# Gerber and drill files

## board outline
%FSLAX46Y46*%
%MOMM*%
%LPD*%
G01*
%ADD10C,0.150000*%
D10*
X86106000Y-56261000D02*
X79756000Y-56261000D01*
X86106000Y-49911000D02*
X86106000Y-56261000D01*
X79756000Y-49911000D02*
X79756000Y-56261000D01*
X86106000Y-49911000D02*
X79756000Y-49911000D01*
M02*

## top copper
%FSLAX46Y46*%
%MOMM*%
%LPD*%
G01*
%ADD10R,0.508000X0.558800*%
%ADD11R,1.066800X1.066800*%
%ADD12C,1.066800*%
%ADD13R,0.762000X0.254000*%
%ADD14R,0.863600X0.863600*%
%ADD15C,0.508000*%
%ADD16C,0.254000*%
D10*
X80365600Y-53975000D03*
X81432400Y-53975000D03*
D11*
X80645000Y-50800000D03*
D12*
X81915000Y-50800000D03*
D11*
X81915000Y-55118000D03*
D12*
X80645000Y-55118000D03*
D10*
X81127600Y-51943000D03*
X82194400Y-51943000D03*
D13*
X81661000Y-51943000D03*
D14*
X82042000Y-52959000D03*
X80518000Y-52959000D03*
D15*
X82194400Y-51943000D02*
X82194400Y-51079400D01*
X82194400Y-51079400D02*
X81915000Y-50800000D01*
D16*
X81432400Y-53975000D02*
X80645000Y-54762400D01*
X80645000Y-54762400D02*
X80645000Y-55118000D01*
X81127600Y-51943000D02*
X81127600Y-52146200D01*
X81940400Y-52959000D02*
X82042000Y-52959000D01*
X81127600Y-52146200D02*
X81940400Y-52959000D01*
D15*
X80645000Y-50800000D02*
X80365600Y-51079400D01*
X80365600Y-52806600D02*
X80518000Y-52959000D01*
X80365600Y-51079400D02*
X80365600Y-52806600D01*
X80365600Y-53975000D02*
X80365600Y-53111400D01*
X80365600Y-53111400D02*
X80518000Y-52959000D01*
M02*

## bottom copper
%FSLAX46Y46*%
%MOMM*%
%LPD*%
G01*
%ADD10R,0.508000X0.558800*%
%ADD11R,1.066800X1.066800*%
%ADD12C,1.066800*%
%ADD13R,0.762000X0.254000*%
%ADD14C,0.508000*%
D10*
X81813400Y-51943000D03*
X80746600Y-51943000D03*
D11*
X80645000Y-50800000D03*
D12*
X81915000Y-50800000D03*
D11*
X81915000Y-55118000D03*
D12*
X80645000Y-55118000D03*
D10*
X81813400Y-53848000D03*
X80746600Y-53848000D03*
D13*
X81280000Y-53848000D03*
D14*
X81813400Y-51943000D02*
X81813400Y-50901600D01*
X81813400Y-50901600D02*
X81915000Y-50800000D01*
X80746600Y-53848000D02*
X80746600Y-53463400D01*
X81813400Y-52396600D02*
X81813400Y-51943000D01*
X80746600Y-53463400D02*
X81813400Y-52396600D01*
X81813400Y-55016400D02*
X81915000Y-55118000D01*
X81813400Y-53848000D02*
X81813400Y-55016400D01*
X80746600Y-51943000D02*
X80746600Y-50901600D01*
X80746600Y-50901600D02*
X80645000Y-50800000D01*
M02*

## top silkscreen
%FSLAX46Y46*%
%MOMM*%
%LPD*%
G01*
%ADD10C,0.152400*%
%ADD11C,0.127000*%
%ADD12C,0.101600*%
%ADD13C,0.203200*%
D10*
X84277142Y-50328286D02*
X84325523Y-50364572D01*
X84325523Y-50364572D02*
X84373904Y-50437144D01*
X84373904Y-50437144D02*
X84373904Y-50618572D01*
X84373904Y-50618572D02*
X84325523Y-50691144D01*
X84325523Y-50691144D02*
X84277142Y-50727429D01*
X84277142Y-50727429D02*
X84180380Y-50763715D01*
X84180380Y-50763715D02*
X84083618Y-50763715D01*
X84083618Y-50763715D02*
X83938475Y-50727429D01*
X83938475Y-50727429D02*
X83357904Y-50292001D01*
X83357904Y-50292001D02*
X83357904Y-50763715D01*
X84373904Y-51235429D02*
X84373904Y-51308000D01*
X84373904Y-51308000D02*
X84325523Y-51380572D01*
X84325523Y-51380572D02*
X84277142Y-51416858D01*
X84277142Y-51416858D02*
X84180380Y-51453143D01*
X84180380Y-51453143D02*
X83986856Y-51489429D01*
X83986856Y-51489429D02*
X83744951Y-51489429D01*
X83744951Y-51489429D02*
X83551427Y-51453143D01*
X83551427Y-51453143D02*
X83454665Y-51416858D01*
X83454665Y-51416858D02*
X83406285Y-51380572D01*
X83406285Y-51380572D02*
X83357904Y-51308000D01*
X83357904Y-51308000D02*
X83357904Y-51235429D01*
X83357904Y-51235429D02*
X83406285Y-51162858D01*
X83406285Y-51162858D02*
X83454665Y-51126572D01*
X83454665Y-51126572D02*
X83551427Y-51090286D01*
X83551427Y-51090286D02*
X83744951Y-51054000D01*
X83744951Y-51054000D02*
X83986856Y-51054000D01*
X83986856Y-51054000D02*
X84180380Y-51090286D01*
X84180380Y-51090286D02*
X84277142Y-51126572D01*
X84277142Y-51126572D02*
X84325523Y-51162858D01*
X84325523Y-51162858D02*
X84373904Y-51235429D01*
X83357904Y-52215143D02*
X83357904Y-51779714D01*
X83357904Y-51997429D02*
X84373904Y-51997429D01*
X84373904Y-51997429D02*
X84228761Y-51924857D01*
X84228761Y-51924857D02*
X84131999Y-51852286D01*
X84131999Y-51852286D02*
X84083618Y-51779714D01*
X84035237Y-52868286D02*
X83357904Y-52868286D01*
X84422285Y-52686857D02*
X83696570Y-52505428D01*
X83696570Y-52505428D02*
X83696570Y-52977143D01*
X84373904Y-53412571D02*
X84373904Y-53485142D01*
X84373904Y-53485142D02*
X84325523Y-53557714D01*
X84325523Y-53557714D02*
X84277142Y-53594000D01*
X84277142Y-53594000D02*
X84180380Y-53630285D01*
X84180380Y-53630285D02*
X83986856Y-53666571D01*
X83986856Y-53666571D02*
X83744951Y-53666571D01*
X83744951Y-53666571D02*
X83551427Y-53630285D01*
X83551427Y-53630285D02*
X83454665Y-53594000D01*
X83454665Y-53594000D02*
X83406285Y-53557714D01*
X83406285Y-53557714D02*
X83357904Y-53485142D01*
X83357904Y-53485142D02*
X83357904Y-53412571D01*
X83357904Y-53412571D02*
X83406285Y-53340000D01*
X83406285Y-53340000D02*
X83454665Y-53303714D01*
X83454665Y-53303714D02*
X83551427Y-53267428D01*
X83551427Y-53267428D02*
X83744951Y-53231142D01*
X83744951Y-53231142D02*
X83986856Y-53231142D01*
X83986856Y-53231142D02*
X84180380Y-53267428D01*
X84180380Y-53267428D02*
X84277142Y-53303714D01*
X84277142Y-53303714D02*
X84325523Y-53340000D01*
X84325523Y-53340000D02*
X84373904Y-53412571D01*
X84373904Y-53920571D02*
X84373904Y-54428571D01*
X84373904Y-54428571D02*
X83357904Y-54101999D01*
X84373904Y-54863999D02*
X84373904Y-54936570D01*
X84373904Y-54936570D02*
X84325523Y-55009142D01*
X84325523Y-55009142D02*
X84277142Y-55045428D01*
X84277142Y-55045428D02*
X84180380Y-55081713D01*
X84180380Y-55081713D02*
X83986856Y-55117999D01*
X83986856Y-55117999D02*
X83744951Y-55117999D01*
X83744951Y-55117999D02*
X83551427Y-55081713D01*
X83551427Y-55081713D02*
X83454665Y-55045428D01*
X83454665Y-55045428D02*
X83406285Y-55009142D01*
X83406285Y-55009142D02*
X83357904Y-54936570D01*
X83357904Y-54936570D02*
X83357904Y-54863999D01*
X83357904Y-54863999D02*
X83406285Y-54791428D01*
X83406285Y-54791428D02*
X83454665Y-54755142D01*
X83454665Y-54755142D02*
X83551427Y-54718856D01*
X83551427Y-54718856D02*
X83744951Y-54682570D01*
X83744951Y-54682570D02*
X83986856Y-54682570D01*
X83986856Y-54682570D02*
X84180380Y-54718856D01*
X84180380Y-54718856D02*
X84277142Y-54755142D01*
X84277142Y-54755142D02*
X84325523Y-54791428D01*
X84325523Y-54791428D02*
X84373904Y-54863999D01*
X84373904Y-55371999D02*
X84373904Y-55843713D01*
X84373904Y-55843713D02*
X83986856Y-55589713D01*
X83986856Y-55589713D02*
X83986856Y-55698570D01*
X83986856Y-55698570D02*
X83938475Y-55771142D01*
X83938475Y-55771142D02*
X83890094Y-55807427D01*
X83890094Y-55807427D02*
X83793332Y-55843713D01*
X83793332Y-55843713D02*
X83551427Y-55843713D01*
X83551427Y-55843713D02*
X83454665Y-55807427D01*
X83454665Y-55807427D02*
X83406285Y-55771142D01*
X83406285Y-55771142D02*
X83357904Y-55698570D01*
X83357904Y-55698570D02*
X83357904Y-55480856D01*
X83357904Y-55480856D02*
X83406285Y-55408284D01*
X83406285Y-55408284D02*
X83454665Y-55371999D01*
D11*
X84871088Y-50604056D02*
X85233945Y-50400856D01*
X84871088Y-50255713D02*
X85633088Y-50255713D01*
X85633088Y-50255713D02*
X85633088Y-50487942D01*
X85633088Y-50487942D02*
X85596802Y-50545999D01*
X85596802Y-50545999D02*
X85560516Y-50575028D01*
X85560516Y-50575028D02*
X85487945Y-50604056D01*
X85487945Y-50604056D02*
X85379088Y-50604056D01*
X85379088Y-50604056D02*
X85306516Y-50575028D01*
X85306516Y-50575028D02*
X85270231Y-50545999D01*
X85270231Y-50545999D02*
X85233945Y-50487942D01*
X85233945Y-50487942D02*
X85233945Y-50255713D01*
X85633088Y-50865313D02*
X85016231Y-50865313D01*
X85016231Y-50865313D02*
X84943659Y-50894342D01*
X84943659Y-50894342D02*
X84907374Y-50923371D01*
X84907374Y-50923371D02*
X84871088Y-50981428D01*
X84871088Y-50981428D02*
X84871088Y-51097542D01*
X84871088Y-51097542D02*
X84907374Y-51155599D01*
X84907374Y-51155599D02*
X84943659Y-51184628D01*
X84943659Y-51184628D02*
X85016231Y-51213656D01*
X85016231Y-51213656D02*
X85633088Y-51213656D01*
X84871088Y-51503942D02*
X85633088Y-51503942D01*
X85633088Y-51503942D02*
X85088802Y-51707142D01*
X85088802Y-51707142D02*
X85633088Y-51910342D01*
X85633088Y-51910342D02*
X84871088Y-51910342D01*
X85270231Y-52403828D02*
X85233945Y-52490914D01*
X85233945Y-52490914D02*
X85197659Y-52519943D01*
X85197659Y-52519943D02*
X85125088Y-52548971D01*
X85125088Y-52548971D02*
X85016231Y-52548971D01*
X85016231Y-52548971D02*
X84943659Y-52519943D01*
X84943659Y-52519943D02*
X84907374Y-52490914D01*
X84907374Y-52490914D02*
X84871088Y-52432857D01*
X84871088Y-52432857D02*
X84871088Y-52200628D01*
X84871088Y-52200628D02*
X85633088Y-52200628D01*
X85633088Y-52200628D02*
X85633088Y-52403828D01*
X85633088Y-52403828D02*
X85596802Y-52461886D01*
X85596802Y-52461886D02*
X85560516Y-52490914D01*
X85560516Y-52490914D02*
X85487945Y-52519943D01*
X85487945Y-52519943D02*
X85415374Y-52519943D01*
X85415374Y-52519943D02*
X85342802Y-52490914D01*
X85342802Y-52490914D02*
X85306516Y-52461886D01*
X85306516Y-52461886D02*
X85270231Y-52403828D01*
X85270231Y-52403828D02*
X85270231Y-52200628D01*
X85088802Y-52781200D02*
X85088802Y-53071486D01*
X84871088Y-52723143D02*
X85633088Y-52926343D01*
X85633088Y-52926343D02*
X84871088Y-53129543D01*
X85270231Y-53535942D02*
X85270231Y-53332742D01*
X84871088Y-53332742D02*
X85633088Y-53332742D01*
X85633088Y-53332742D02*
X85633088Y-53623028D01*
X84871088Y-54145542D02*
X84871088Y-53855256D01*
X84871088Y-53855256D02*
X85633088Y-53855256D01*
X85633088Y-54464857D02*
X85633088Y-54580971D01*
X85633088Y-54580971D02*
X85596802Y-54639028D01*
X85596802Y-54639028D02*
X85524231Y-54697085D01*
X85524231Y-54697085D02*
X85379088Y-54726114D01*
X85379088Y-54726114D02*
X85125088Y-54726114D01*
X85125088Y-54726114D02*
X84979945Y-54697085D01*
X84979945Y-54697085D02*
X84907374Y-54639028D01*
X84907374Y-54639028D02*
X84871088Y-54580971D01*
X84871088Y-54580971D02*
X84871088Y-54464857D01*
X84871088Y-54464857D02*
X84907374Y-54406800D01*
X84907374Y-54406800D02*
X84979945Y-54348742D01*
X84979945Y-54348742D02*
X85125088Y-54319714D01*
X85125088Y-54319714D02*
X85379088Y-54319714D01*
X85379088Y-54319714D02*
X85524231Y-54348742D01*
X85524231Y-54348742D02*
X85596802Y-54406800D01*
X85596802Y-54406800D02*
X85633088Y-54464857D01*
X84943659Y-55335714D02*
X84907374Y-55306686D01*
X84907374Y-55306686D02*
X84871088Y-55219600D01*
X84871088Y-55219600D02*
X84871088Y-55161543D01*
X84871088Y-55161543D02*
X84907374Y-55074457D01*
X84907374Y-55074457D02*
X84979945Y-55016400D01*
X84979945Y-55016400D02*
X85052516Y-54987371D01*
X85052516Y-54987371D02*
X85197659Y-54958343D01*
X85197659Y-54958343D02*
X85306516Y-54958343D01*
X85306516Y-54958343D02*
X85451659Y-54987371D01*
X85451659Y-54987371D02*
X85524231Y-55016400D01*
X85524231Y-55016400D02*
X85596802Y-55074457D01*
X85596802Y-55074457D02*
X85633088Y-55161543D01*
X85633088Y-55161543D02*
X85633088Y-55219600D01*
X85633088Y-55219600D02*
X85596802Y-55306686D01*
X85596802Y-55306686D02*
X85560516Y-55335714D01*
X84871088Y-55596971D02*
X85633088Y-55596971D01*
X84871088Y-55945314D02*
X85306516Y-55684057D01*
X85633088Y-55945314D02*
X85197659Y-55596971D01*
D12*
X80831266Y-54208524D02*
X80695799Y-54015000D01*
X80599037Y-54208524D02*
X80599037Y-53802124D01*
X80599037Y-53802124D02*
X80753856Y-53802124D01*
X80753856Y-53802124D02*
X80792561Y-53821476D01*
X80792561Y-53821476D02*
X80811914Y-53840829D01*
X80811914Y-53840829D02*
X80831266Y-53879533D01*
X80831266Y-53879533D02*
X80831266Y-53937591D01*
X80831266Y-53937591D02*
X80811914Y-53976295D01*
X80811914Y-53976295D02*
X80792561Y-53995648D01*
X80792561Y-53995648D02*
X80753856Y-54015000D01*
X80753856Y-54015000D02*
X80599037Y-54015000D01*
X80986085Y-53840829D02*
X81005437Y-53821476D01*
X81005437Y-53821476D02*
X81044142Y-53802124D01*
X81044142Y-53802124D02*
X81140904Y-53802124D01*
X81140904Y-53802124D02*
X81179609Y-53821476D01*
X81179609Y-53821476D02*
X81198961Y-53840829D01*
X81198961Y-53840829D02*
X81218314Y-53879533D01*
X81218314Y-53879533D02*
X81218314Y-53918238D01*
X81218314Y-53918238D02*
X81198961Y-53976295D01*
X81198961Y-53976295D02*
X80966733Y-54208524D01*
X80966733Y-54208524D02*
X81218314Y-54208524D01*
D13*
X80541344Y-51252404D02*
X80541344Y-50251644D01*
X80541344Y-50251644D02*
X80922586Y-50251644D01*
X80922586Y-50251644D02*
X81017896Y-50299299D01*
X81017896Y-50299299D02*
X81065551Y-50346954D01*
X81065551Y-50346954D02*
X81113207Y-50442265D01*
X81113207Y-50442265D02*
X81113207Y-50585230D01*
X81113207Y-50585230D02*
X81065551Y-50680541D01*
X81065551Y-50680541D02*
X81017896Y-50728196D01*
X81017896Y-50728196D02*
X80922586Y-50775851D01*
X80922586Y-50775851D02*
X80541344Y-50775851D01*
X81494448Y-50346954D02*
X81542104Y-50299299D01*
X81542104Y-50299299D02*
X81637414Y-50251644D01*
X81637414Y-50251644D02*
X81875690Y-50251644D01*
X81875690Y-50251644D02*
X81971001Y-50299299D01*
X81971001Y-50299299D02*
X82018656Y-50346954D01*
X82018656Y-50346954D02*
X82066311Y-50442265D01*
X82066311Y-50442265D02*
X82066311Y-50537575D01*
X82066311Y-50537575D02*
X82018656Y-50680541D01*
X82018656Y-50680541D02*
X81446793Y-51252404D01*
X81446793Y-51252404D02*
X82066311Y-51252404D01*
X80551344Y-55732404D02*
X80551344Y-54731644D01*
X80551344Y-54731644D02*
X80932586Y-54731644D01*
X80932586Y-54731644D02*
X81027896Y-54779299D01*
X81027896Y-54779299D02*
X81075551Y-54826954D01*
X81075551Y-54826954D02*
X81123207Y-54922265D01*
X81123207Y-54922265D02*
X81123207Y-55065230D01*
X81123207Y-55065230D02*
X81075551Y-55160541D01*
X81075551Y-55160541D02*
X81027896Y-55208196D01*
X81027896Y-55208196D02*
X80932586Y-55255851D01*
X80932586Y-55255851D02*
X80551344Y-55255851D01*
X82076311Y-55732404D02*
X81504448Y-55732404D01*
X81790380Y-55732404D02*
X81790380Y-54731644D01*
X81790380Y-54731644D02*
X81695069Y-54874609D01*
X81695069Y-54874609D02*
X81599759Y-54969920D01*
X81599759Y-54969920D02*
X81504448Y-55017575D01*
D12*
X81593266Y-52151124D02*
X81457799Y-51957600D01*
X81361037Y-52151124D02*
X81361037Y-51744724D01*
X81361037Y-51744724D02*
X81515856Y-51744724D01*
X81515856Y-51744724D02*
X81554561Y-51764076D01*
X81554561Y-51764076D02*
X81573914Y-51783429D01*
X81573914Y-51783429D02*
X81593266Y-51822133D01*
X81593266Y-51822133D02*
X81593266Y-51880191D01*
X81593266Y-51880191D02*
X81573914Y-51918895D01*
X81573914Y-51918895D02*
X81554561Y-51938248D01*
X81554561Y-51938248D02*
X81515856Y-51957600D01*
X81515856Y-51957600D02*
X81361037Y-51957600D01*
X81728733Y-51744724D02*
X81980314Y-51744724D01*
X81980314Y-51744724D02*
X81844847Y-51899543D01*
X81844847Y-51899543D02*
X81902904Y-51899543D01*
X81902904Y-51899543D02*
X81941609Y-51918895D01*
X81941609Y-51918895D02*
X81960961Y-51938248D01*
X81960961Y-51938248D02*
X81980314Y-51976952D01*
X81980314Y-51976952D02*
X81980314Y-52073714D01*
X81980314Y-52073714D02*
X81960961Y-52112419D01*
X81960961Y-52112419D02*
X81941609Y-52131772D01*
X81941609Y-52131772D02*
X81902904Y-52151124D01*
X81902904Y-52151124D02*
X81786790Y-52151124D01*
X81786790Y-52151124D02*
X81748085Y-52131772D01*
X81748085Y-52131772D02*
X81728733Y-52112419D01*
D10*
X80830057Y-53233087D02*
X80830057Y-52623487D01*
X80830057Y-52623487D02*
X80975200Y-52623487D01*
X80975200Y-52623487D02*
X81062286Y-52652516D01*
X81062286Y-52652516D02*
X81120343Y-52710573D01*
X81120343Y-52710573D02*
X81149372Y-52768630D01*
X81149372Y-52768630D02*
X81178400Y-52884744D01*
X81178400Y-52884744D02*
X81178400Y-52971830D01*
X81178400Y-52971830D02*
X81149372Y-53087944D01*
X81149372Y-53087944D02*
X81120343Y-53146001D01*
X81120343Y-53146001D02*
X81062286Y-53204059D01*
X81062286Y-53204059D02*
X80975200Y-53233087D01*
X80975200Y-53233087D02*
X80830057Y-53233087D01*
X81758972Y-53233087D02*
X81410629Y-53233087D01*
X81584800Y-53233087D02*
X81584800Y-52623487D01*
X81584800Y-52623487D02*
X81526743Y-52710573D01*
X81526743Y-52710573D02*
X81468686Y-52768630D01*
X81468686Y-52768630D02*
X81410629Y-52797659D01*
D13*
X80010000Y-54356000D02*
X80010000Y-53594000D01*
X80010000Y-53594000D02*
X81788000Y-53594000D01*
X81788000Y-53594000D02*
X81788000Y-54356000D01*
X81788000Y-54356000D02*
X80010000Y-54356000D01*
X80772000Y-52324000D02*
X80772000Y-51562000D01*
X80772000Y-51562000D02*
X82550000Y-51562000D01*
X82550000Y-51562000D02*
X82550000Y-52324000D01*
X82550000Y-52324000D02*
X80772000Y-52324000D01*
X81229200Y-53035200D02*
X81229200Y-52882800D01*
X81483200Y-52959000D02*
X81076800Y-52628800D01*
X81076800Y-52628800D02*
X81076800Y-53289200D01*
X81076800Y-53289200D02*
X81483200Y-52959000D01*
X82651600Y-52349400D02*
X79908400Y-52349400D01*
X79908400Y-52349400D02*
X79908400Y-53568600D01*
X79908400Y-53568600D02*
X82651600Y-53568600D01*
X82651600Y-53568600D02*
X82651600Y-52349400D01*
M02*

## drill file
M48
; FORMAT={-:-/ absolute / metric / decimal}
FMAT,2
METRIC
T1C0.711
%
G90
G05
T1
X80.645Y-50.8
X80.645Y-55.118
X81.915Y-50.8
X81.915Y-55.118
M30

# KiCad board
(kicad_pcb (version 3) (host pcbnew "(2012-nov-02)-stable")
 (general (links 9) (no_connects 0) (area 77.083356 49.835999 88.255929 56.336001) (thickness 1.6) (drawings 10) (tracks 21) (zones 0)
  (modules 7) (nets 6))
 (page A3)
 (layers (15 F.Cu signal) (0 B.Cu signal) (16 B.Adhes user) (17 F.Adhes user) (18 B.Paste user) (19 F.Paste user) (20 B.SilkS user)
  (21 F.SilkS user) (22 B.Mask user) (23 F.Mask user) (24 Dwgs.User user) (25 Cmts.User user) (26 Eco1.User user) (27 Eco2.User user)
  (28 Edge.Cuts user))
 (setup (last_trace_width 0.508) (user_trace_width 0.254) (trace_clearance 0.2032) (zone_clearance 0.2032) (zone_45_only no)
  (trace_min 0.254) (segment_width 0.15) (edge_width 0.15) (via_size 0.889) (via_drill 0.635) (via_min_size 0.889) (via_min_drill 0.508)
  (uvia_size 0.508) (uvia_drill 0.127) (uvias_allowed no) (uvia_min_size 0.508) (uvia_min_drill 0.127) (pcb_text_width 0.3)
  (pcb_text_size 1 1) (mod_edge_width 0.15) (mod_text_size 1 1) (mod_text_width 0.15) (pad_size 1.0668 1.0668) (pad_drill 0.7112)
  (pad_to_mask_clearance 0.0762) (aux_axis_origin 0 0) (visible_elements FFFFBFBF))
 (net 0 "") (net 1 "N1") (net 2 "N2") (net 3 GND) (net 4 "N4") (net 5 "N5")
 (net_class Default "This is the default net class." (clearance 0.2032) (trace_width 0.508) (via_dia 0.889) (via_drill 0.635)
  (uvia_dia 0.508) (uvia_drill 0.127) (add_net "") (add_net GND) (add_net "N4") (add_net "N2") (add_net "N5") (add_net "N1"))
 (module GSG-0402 (layer F.Cu) (at 80.899 53.975 180) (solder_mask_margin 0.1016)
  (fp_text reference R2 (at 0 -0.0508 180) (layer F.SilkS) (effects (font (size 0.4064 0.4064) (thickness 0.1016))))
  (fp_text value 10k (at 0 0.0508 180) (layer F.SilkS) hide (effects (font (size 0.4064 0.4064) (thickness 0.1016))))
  (fp_line (start 0.889 -0.381) (end 0.889 0.381) (layer F.SilkS) (width 0.2032))
  (fp_line (start 0.889 0.381) (end -0.889 0.381) (layer F.SilkS) (width 0.2032))
  (fp_line (start -0.889 0.381) (end -0.889 -0.381) (layer F.SilkS) (width 0.2032))
  (fp_line (start -0.889 -0.381) (end 0.889 -0.381) (layer F.SilkS) (width 0.2032))
  (pad 2 smd rect (at 0.5334 0 180) (size 0.508 0.5588) (layers F.Cu F.Paste F.Mask) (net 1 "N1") (solder_mask_margin 0.1016))
  (pad 1 smd rect (at -0.5334 0 180) (size 0.508 0.5588) (layers F.Cu F.Paste F.Mask) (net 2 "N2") (die_length -2147.483648)
   (solder_mask_margin 0.1016)))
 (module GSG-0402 (layer B.Cu) (at 81.28 51.943) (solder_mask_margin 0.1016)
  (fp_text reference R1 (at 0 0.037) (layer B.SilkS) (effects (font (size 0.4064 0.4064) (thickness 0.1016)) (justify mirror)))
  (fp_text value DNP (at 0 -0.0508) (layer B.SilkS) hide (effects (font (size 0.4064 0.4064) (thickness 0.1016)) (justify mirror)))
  (pad 2 smd rect (at 0.5334 0) (size 0.508 0.5588) (layers B.Cu B.Paste B.Mask) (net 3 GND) (solder_mask_margin 0.1016))
  (pad 1 smd rect (at -0.5334 0) (size 0.508 0.5588) (layers B.Cu B.Paste B.Mask) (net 1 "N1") (die_length -2147.483648)
   (solder_mask_margin 0.1016)))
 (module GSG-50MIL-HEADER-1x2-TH (layer F.Cu) (at 81.28 50.8)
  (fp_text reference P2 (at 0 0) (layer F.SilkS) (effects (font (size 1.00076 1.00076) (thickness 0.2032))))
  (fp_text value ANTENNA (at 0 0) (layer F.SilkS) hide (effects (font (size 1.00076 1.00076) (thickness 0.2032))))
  (pad 1 thru_hole rect (at -0.635 0) (size 1.0668 1.0668) (drill 0.7112) (layers *.Cu *.Mask) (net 1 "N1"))
  (pad 2 thru_hole circle (at 0.635 0) (size 1.0668 1.0668) (drill 0.7112) (layers *.Cu *.Mask) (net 3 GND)))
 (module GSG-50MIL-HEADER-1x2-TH (layer F.Cu) (at 81.28 55.118 180)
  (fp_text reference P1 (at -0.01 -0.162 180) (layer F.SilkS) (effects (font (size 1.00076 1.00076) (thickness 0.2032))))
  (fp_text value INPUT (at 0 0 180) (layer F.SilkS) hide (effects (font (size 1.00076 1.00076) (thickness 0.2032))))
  (pad 1 thru_hole rect (at -0.635 0 180) (size 1.0668 1.0668) (drill 0.7112) (layers *.Cu *.Mask) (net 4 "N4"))
  (pad 2 thru_hole circle (at 0.635 0 180) (size 1.0668 1.0668) (drill 0.7112) (layers *.Cu *.Mask) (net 2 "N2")))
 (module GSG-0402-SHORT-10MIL (layer B.Cu) (at 81.28 53.848) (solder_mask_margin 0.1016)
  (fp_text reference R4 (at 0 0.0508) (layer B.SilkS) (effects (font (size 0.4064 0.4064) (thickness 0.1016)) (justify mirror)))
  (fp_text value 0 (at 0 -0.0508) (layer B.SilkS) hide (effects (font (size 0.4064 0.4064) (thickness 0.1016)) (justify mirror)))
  (pad 2 smd rect (at 0.5334 0) (size 0.508 0.5588) (layers B.Cu B.Mask) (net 4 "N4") (solder_mask_margin 0.1016))
  (pad 1 smd rect (at -0.5334 0) (size 0.508 0.5588) (layers B.Cu B.Mask) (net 3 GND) (die_length -2147.483648) (solder_mask_margin 0.1016))
  (pad "" smd rect (at 0 0) (size 0.762 0.254) (layers B.Cu B.Mask)))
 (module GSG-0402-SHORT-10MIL (layer F.Cu) (at 81.661 51.943 180) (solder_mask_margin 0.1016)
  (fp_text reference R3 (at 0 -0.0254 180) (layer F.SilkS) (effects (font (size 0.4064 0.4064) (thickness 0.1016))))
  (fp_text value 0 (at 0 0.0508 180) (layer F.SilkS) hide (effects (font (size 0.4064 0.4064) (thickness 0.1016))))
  (fp_line (start 0.889 -0.381) (end 0.889 0.381) (layer F.SilkS) (width 0.2032))
  (fp_line (start 0.889 0.381) (end -0.889 0.381) (layer F.SilkS) (width 0.2032))
  (fp_line (start -0.889 0.381) (end -0.889 -0.381) (layer F.SilkS) (width 0.2032))
  (fp_line (start -0.889 -0.381) (end 0.889 -0.381) (layer F.SilkS) (width 0.2032))
  (pad 2 smd rect (at 0.5334 0 180) (size 0.508 0.5588) (layers F.Cu F.Mask) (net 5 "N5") (solder_mask_margin 0.1016))
  (pad 1 smd rect (at -0.5334 0 180) (size 0.508 0.5588) (layers F.Cu F.Mask) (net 3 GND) (die_length -2147.483648)
   (solder_mask_margin 0.1016))
  (pad "" smd rect (at 0 0 180) (size 0.762 0.254) (layers F.Cu F.Mask)))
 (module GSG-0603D (layer F.Cu) (at 81.28 52.959) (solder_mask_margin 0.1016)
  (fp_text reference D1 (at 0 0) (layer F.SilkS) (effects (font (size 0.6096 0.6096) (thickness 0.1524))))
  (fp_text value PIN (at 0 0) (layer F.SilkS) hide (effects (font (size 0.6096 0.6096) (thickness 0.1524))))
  (fp_line (start -0.0508 0.0762) (end -0.0508 -0.0762) (layer F.SilkS) (width 0.2032))
  (fp_line (start 0.2032 0) (end -0.2032 -0.3302) (layer F.SilkS) (width 0.2032))
  (fp_line (start -0.2032 -0.3302) (end -0.2032 0.3302) (layer F.SilkS) (width 0.2032))
  (fp_line (start -0.2032 0.3302) (end 0.2032 0) (layer F.SilkS) (width 0.2032))
  (fp_line (start 1.3716 -0.6096) (end -1.3716 -0.6096) (layer F.SilkS) (width 0.2032))
  (fp_line (start -1.3716 -0.6096) (end -1.3716 0.6096) (layer F.SilkS) (width 0.2032))
  (fp_line (start -1.3716 0.6096) (end 1.3716 0.6096) (layer F.SilkS) (width 0.2032))
  (fp_line (start 1.3716 0.6096) (end 1.3716 -0.6096) (layer F.SilkS) (width 0.2032))
  (pad 2 smd rect (at 0.762 0) (size 0.8636 0.8636) (layers F.Cu F.Paste F.Mask) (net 5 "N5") (die_length 0.04572)
   (solder_mask_margin 0.1016) (clearance 0.1778))
  (pad 1 smd rect (at -0.762 0) (size 0.8636 0.8636) (layers F.Cu F.Paste F.Mask) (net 1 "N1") (die_length 0.08382)
   (solder_mask_margin 0.1016) (clearance 0.1778)))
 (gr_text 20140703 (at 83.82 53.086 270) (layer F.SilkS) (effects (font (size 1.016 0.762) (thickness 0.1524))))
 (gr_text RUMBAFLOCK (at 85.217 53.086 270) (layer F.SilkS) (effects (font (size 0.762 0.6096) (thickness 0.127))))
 (gr_line (start 86.106 56.261) (end 79.756 56.261) (angle 90) (layer Edge.Cuts) (width 0.15))
 (gr_line (start 86.106 49.911) (end 86.106 56.261) (angle 90) (layer Edge.Cuts) (width 0.15))
 (gr_line (start 79.756 49.911) (end 79.756 56.261) (angle 90) (layer Edge.Cuts) (width 0.15))
 (gr_line (start 86.106 49.911) (end 79.756 49.911) (angle 90) (layer Edge.Cuts) (width 0.15))
 (segment (start 82.1944 51.943) (end 82.1944 51.0794) (width 0.508) (layer F.Cu) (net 3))
 (segment (start 82.1944 51.0794) (end 81.915 50.8) (width 0.508) (layer F.Cu) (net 3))
 (segment (start 81.8134 51.943) (end 81.8134 50.9016) (width 0.508) (layer B.Cu) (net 3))
 (segment (start 81.8134 50.9016) (end 81.915 50.8) (width 0.508) (layer B.Cu) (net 3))
 (segment (start 80.7466 53.848) (end 80.7466 53.4634) (width 0.508) (layer B.Cu) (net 3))
 (segment (start 81.8134 52.3966) (end 81.8134 51.943) (width 0.508) (layer B.Cu) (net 3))
 (segment (start 80.7466 53.4634) (end 81.8134 52.3966) (width 0.508) (layer B.Cu) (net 3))
 (segment (start 81.8134 55.0164) (end 81.915 55.118) (width 0.508) (layer B.Cu) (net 4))
 (segment (start 81.8134 53.848) (end 81.8134 55.0164) (width 0.508) (layer B.Cu) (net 4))
 (segment (start 81.4324 53.975) (end 80.645 54.7624) (width 0.254) (layer F.Cu) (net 2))
 (segment (start 80.645 54.7624) (end 80.645 55.118) (width 0.254) (layer F.Cu) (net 2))
 (segment (start 81.1276 51.943) (end 81.1276 52.1462) (width 0.254) (layer F.Cu) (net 5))
 (segment (start 81.9404 52.959) (end 82.042 52.959) (width 0.254) (layer F.Cu) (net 5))
 (segment (start 81.1276 52.1462) (end 81.9404 52.959) (width 0.254) (layer F.Cu) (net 5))
 (segment (start 80.645 50.8) (end 80.3656 51.0794) (width 0.508) (layer F.Cu) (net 1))
 (segment (start 80.3656 52.8066) (end 80.518 52.959) (width 0.508) (layer F.Cu) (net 1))
 (segment (start 80.3656 51.0794) (end 80.3656 52.8066) (width 0.508) (layer F.Cu) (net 1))
 (segment (start 80.3656 53.975) (end 80.3656 53.1114) (width 0.508) (layer F.Cu) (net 1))
 (segment (start 80.3656 53.1114) (end 80.518 52.959) (width 0.508) (layer F.Cu) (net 1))
 (segment (start 80.7466 51.943) (end 80.7466 50.9016) (width 0.508) (layer B.Cu) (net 1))
 (segment (start 80.7466 50.9016) (end 80.645 50.8) (width 0.508) (layer B.Cu) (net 1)))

